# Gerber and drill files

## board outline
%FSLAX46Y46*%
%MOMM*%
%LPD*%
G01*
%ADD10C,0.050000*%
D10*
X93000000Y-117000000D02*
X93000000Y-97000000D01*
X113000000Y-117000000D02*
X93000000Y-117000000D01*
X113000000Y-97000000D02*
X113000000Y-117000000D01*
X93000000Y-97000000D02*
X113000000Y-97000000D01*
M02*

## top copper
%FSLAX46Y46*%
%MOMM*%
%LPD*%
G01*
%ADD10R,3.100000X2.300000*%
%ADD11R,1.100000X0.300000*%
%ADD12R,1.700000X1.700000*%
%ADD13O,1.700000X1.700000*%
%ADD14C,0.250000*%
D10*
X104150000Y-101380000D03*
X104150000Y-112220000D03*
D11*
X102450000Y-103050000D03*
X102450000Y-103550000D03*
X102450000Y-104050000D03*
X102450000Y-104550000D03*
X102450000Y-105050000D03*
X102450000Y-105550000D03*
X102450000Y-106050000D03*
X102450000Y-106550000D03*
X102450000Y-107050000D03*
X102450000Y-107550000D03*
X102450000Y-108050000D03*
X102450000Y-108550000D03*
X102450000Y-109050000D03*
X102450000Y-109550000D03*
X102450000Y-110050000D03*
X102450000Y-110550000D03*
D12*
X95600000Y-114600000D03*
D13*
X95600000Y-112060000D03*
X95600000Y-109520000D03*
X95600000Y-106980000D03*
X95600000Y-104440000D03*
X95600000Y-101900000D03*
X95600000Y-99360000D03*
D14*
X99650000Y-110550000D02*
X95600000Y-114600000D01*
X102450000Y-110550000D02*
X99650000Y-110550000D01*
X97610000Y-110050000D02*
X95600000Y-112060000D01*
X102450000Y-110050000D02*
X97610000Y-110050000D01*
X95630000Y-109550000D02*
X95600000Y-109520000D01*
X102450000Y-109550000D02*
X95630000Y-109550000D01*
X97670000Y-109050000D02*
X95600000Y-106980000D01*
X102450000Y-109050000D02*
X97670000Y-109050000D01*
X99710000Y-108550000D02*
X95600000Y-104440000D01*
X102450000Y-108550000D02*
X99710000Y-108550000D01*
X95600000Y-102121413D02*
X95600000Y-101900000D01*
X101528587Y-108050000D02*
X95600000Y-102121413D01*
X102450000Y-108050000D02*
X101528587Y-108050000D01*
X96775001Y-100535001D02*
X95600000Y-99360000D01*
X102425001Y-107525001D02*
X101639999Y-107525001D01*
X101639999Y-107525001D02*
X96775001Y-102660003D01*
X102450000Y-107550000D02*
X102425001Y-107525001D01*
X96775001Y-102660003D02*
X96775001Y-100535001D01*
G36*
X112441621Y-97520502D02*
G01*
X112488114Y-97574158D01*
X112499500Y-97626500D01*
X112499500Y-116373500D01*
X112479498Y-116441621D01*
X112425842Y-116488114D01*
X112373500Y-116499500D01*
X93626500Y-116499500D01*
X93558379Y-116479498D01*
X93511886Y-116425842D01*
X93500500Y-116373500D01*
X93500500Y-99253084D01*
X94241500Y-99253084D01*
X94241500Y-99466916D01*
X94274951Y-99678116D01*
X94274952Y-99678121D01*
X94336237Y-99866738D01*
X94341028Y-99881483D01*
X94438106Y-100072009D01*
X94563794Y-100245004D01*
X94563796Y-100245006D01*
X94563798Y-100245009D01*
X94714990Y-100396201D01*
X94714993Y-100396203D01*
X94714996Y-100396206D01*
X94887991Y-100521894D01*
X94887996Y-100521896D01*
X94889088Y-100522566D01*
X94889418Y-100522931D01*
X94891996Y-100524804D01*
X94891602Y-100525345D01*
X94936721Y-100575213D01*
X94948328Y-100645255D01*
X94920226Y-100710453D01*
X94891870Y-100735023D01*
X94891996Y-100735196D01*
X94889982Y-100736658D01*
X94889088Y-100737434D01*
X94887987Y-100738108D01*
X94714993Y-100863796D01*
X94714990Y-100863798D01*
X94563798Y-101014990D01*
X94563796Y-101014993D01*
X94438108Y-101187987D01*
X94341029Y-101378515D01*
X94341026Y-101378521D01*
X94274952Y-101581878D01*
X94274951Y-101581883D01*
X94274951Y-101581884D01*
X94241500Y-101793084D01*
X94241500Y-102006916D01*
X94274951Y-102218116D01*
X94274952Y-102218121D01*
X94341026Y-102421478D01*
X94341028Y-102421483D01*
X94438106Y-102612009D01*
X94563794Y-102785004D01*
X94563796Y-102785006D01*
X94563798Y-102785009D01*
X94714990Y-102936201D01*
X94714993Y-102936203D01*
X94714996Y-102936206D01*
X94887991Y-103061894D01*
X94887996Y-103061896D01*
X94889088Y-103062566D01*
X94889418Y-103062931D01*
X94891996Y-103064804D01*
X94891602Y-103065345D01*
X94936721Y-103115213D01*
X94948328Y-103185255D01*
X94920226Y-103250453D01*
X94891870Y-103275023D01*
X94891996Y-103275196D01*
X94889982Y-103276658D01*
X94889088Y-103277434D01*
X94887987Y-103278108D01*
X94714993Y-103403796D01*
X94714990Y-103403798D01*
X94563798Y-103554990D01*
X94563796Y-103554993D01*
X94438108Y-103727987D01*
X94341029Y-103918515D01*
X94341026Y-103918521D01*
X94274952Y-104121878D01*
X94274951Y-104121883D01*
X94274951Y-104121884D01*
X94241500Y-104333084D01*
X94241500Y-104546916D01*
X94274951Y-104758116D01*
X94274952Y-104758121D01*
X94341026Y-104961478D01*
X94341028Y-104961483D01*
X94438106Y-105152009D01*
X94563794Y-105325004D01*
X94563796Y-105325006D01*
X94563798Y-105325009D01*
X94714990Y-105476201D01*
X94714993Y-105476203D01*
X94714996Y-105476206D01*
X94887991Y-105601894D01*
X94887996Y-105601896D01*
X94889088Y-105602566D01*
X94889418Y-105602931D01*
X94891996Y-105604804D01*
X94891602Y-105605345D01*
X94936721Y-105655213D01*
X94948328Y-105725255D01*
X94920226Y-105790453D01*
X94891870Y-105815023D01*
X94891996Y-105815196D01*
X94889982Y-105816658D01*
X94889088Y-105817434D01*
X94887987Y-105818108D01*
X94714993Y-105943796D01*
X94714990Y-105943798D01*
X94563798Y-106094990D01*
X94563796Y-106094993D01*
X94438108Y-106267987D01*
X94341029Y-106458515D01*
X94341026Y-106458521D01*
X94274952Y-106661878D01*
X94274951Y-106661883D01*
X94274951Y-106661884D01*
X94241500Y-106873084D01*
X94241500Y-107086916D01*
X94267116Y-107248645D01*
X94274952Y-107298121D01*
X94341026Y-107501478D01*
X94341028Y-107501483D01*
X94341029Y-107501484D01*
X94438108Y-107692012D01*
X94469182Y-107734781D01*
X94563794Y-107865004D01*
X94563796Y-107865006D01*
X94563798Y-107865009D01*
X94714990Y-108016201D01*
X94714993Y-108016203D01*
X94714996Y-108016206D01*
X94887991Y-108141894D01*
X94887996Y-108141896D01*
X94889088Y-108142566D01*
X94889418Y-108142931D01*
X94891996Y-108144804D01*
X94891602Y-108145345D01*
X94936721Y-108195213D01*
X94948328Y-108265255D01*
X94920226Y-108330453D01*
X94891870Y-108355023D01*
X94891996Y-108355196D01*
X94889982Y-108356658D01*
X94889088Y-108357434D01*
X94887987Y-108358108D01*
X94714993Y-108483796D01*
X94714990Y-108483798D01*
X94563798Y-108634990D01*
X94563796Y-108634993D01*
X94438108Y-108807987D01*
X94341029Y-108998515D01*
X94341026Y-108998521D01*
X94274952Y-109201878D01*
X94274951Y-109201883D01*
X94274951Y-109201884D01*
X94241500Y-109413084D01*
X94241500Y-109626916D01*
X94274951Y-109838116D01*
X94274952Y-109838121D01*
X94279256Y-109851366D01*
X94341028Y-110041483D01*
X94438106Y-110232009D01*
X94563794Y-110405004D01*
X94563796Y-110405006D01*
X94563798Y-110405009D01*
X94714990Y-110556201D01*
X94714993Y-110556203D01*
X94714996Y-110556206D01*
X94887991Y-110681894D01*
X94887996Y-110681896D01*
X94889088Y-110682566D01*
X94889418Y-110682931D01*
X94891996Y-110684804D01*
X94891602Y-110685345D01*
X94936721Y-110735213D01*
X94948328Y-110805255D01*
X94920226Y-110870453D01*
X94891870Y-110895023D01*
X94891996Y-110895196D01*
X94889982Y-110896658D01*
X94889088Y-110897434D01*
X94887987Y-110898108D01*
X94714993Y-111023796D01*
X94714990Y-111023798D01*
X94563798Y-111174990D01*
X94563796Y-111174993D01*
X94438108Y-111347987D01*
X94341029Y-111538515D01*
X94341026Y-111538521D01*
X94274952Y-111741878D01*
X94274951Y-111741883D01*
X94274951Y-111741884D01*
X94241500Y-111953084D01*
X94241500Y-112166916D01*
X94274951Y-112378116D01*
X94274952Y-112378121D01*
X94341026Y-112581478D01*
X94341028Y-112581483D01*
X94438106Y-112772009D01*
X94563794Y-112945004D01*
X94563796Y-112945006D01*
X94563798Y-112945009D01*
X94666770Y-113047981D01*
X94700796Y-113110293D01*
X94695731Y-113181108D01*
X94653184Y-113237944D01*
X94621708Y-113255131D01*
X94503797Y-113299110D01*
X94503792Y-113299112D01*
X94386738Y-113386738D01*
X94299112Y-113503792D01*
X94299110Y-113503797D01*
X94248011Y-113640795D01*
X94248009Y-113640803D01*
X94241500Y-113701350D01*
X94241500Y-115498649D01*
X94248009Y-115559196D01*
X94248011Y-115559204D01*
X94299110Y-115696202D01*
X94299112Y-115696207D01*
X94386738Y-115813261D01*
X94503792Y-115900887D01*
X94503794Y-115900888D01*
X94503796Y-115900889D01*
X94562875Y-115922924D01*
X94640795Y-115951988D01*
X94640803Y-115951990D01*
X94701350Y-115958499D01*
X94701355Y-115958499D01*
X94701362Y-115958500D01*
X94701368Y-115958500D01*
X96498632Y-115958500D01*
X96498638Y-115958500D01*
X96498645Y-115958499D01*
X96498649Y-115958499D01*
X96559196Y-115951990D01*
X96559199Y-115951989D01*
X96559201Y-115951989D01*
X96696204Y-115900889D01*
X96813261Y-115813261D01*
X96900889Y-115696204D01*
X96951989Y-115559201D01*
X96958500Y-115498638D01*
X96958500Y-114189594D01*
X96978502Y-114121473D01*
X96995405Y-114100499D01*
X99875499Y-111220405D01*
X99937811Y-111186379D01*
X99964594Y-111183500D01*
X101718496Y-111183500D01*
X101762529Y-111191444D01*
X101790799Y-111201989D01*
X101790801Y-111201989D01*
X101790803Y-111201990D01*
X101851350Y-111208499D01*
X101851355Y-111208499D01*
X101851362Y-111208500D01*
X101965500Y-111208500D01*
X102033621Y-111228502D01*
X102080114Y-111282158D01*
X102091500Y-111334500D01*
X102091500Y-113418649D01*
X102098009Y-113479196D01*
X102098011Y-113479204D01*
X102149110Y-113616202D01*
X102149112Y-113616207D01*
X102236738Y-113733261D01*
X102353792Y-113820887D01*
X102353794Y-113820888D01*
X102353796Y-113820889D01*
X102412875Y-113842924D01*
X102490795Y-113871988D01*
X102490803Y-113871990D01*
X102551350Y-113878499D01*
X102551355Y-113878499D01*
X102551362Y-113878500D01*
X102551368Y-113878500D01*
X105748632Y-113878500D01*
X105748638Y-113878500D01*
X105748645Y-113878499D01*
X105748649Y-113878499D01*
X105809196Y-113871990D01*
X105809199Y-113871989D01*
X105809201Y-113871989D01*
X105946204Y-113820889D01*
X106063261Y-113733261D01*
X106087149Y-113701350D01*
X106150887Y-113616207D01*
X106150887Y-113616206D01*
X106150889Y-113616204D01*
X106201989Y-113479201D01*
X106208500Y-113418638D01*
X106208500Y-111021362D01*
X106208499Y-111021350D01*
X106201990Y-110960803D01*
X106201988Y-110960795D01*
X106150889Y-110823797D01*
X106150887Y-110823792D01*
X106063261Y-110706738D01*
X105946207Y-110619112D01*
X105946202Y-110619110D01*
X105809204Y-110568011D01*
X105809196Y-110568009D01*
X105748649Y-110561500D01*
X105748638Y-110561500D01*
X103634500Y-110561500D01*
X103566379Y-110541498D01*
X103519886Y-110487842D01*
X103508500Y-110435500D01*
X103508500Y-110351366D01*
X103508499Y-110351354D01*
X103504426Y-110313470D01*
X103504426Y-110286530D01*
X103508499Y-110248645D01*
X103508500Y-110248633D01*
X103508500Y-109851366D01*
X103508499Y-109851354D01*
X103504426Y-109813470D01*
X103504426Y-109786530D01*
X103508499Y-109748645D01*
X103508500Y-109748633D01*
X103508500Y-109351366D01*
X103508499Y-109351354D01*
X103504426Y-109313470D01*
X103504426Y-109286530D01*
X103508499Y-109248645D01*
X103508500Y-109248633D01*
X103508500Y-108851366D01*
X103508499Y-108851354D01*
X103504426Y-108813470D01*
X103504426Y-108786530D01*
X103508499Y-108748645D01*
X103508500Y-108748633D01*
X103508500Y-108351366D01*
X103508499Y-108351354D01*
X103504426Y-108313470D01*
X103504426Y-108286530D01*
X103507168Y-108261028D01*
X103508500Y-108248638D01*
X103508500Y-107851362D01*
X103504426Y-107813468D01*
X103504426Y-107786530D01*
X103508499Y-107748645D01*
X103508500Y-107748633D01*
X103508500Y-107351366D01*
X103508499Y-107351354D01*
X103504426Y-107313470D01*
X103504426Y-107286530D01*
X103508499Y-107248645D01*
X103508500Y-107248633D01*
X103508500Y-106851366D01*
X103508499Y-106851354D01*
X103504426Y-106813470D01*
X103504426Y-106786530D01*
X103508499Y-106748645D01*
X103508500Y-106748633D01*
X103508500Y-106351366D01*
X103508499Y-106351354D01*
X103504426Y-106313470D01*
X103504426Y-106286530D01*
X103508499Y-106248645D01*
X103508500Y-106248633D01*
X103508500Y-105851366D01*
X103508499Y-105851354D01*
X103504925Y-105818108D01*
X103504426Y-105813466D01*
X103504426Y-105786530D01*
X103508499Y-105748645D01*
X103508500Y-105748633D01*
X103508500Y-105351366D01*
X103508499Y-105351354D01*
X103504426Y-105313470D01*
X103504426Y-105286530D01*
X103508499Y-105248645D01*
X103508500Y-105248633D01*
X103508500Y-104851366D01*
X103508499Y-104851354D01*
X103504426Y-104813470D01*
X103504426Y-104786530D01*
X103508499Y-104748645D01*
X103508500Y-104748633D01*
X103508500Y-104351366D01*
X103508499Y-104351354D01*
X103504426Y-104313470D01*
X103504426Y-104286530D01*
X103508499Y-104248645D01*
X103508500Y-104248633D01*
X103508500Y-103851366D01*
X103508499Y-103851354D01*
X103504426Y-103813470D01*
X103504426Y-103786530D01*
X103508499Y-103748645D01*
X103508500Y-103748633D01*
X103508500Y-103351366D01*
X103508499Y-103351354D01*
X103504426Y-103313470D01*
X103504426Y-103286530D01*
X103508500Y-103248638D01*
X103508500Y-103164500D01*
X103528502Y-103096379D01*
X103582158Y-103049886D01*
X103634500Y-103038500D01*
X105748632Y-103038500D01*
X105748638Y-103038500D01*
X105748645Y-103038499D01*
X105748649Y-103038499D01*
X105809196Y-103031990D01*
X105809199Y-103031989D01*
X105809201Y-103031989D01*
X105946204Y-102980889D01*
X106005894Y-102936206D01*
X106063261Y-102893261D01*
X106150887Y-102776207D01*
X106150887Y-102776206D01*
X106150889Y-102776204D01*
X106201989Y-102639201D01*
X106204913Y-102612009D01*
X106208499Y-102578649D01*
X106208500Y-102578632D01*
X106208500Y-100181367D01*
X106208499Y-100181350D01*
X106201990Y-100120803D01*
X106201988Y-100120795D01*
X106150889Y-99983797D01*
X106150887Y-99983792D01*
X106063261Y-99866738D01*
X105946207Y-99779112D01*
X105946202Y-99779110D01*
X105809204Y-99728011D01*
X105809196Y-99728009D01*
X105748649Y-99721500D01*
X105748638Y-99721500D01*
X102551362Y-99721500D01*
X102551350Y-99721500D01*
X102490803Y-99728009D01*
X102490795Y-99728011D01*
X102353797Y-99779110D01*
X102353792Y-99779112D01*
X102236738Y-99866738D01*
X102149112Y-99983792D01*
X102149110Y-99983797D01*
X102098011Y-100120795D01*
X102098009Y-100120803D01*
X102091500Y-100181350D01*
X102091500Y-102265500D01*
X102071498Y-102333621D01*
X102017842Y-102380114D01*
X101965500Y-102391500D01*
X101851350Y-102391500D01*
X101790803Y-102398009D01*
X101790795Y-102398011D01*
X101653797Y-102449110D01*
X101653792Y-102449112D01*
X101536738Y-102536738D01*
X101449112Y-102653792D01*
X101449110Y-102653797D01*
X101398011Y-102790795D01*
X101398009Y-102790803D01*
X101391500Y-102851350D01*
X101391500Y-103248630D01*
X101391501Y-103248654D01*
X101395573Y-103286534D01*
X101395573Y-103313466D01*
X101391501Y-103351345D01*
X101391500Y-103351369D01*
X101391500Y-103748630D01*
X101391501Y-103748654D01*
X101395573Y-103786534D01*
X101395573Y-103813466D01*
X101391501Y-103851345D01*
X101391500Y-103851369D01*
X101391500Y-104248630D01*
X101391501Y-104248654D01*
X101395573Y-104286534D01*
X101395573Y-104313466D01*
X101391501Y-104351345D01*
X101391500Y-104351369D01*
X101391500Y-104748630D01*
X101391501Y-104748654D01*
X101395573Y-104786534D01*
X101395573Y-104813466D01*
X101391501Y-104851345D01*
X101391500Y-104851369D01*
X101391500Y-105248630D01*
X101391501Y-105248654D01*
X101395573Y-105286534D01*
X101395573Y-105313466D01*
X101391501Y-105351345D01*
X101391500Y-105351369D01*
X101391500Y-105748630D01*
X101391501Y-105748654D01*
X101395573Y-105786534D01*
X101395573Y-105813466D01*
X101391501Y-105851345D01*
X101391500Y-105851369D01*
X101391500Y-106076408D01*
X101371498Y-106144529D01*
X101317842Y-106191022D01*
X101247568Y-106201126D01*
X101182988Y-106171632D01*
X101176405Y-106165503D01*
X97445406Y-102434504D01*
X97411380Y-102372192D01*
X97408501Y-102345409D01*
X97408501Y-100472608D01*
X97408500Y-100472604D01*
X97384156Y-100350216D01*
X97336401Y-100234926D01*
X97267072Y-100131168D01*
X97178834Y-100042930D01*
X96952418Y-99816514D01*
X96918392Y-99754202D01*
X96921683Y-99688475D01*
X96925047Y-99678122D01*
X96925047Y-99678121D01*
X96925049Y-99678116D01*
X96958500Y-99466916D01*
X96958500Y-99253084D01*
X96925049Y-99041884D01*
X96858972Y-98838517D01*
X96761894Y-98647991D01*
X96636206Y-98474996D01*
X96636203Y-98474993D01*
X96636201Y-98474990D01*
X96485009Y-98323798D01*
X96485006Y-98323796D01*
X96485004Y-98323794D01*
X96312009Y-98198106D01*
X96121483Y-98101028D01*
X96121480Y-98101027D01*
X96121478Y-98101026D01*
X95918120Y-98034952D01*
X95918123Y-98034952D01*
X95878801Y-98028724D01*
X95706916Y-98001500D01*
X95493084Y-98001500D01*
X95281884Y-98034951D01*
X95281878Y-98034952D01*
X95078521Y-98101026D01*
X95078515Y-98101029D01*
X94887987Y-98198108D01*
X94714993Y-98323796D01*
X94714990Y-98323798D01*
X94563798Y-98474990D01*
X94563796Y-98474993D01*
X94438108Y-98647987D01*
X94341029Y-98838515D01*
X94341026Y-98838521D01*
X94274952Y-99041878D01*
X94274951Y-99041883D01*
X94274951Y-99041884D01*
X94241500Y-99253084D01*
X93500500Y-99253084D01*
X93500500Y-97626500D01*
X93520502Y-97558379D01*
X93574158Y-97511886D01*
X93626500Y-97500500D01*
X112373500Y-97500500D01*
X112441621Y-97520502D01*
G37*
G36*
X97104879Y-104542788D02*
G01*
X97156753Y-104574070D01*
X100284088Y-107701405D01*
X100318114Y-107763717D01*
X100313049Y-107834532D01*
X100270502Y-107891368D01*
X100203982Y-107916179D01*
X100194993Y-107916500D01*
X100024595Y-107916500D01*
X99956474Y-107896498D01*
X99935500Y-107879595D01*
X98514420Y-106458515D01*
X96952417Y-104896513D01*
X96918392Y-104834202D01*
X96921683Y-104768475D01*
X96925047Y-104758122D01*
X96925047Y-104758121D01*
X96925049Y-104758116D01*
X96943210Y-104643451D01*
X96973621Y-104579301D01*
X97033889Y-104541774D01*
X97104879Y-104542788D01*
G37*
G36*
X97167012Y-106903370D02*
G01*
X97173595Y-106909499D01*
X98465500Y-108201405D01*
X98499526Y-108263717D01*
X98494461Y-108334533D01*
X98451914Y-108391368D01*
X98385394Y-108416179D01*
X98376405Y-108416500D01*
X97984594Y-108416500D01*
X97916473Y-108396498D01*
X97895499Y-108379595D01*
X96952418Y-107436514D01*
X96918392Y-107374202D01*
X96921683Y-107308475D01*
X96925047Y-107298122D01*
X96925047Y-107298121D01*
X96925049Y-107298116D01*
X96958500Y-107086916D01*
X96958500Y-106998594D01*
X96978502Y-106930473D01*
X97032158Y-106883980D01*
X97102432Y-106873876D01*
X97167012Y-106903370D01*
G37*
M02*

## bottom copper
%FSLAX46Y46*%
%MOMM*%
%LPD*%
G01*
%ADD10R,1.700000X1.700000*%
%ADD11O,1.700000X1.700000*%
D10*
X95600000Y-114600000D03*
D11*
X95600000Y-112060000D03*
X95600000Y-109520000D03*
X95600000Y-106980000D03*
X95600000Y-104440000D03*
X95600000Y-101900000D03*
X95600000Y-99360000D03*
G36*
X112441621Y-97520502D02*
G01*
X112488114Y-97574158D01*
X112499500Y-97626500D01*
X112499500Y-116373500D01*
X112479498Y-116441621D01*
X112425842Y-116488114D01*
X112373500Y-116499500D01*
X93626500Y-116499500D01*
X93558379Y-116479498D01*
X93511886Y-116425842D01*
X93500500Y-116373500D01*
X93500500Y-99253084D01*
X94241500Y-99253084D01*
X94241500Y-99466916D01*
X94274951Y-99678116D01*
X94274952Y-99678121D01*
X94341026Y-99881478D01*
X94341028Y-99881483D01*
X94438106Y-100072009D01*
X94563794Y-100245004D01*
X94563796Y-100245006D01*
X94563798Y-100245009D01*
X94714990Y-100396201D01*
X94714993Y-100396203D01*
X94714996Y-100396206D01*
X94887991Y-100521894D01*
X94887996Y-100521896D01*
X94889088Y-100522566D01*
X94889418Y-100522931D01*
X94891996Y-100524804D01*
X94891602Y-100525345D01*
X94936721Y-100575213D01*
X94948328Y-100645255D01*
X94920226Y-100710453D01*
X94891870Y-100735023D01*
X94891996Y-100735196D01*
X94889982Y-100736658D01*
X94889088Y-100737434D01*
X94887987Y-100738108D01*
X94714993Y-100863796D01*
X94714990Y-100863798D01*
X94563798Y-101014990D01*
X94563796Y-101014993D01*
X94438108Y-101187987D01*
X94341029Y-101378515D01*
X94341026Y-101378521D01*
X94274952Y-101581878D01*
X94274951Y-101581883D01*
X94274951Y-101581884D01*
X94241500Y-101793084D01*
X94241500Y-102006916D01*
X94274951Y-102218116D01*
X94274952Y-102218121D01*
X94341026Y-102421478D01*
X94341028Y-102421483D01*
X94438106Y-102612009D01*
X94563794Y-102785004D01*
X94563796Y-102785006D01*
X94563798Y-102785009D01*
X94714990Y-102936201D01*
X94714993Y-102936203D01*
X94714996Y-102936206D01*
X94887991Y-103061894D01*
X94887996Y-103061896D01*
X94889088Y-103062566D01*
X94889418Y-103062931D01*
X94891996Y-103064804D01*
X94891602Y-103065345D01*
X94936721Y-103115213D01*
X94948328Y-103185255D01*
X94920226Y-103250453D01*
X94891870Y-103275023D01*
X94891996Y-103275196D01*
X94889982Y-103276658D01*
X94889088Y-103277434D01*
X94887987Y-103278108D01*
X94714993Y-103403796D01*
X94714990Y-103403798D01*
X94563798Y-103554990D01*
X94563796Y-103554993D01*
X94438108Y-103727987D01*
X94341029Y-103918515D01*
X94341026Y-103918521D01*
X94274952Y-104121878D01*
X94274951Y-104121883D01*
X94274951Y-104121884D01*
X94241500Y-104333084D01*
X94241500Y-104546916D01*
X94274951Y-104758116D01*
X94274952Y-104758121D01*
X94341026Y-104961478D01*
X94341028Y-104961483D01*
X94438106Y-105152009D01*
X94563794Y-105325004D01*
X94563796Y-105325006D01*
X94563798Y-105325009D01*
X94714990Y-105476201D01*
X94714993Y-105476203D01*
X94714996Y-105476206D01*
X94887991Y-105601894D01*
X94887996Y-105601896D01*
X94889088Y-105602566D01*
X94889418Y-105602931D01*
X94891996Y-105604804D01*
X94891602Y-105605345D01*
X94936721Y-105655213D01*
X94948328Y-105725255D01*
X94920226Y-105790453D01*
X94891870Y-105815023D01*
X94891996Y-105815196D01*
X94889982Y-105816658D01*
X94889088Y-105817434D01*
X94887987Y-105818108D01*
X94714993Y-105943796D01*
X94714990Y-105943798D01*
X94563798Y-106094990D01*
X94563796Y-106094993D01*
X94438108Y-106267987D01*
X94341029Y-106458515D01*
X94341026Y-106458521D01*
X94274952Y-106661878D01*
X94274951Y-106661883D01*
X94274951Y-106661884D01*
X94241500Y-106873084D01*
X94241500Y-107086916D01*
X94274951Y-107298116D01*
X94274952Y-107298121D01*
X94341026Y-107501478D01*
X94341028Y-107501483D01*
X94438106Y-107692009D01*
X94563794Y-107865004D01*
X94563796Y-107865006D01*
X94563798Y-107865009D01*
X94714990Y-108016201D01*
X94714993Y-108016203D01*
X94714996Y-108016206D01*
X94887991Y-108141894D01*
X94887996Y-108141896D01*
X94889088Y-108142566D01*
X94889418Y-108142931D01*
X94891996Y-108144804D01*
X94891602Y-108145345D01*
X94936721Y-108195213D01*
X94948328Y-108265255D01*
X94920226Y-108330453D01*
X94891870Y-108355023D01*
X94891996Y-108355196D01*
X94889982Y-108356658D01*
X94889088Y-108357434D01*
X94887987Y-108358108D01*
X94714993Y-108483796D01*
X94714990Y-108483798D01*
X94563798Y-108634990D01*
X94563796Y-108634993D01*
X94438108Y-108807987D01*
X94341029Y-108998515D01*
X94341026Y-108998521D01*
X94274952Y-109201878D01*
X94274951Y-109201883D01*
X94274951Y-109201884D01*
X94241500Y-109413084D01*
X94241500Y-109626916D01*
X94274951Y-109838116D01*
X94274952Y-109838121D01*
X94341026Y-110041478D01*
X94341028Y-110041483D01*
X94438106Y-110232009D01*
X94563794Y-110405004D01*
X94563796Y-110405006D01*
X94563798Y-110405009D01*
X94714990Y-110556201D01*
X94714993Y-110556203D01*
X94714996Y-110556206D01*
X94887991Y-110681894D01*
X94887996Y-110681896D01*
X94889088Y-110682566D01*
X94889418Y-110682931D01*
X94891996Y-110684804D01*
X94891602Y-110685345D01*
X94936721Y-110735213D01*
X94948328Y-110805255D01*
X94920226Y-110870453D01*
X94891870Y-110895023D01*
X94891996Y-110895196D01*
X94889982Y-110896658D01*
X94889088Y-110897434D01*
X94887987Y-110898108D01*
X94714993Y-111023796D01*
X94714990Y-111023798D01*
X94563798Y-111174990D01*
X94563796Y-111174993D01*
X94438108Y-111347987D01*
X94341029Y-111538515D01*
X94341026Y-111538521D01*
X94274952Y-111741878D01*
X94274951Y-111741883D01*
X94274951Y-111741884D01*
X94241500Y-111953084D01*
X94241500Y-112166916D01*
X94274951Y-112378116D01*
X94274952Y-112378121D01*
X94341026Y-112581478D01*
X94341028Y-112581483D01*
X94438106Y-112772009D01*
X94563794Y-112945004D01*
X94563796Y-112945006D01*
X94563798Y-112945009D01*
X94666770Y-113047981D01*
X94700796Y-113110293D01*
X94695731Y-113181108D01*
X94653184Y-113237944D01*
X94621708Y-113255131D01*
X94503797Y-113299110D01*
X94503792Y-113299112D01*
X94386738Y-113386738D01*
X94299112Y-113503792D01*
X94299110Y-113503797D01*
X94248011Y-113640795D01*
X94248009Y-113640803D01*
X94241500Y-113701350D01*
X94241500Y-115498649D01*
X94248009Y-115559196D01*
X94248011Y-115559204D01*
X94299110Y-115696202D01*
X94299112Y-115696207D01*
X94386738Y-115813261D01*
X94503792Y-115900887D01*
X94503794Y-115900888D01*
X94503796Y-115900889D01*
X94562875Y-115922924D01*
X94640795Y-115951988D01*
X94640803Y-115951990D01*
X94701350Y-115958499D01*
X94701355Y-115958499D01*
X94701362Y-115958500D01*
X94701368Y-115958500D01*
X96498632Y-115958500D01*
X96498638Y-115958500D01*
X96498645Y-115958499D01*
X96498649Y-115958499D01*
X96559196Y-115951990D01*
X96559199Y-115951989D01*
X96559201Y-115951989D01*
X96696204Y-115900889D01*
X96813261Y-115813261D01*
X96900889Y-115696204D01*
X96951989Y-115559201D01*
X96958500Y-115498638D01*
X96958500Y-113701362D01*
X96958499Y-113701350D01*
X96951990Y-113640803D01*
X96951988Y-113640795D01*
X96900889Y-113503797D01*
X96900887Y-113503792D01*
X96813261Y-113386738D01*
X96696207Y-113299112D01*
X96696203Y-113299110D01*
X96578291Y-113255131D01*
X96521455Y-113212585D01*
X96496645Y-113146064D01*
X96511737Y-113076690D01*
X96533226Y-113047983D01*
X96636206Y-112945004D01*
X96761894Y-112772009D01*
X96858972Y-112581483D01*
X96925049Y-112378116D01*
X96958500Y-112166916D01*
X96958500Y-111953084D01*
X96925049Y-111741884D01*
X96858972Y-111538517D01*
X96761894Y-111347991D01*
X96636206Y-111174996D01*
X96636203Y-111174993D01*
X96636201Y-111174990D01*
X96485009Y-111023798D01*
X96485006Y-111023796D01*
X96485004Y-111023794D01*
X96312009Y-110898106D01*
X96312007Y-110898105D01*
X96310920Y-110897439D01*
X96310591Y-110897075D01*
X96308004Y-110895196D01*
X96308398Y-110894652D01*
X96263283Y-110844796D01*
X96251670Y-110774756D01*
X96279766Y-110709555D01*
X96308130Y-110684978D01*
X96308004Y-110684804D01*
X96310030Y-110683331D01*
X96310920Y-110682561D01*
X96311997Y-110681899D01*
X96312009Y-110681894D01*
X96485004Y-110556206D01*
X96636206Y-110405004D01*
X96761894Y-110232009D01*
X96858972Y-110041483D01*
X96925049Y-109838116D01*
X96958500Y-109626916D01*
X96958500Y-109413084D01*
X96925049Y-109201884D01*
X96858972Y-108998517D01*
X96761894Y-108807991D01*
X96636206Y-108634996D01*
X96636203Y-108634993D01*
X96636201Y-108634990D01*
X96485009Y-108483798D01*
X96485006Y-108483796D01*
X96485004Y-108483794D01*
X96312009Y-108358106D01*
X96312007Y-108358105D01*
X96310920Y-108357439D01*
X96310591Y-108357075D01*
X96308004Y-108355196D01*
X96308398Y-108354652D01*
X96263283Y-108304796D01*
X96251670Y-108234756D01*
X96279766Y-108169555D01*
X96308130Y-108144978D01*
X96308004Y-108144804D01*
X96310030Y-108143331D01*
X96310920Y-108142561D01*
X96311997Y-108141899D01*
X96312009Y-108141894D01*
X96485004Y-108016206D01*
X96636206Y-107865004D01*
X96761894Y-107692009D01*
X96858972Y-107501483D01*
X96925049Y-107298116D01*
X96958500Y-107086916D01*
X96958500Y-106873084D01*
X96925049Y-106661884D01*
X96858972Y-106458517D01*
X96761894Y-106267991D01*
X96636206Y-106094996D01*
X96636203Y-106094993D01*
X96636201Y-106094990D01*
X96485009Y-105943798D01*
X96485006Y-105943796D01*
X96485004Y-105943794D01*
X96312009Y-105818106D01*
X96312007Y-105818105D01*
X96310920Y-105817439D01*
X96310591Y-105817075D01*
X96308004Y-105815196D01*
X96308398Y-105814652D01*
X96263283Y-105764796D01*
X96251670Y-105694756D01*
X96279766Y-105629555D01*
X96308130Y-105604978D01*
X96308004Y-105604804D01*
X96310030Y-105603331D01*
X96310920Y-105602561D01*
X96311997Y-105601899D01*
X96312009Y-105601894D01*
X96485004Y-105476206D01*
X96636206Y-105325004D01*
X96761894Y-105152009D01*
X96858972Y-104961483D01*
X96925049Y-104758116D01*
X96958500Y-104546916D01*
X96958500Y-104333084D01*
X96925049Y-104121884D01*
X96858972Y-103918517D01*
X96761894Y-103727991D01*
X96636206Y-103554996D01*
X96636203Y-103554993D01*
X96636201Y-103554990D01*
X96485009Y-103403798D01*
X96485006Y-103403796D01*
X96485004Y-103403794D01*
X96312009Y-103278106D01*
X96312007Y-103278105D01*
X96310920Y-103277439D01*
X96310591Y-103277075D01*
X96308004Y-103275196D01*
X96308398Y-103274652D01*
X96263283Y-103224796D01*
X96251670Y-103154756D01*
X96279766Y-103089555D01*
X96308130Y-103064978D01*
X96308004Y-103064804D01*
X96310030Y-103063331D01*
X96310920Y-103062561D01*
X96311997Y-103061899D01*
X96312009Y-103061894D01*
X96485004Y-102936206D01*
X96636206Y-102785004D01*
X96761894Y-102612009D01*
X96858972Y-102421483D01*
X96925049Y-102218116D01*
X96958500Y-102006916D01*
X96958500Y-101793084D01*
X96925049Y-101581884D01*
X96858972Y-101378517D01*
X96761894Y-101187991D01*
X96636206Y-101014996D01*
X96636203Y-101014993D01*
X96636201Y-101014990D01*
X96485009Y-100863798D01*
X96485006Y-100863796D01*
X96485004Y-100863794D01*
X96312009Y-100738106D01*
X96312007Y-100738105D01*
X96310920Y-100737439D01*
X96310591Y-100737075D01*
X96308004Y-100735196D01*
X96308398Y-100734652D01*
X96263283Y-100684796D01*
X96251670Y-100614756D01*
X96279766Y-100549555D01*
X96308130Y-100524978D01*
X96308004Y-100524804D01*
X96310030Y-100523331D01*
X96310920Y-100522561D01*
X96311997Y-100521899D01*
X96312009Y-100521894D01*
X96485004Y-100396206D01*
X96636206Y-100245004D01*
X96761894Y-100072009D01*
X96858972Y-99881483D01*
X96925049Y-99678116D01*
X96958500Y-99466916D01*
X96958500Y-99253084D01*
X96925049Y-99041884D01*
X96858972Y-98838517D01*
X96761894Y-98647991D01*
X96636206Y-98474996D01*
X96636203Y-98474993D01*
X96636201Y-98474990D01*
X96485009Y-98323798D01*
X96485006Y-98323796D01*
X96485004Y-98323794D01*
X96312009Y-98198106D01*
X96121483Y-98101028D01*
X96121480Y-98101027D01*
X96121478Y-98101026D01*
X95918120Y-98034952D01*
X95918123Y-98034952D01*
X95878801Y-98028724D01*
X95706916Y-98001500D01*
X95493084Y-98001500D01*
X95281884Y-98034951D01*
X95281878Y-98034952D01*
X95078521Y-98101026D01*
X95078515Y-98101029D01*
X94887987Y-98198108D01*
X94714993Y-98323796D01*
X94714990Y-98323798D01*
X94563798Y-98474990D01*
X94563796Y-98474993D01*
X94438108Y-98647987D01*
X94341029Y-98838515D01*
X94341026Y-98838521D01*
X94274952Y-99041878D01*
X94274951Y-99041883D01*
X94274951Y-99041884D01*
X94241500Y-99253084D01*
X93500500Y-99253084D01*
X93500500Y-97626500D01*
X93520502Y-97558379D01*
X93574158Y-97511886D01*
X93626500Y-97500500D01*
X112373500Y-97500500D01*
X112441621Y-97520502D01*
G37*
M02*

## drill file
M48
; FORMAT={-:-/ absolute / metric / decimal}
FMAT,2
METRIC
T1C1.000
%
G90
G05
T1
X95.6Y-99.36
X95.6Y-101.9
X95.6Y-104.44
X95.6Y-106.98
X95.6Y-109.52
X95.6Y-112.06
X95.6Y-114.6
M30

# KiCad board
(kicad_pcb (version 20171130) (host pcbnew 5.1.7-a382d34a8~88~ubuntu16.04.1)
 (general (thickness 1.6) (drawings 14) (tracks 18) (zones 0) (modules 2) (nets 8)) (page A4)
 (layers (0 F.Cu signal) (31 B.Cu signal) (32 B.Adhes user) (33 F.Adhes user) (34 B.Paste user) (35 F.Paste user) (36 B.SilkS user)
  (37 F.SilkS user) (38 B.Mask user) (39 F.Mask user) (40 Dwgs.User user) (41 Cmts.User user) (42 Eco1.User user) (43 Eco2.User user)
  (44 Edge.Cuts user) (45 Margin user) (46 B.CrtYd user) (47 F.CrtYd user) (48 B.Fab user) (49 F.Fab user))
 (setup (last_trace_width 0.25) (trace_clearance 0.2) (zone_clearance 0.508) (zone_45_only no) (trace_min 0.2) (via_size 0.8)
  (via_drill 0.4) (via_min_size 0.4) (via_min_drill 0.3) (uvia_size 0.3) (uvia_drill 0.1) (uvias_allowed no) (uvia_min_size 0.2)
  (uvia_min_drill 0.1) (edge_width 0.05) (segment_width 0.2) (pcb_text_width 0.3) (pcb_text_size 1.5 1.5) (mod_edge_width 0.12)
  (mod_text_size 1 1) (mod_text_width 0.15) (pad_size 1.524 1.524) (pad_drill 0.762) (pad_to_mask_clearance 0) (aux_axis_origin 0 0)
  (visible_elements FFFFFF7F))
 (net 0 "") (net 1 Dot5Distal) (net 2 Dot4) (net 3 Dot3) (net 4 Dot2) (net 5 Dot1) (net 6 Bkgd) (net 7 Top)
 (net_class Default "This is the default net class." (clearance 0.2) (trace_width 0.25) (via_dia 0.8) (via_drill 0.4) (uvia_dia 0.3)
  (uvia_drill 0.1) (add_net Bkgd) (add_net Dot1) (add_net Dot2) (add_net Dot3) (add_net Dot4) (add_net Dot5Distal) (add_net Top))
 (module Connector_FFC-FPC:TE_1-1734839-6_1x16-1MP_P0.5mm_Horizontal (layer F.Cu) (at 103.8 106.8 90)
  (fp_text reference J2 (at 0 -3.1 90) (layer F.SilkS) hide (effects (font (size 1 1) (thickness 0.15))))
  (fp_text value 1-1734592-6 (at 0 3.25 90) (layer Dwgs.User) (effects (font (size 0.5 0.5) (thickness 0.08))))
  (pad MP smd rect (at 5.42 0.35 90) (size 2.3 3.1) (layers F.Cu F.Paste F.Mask))
  (pad MP smd rect (at -5.42 0.35 90) (size 2.3 3.1) (layers F.Cu F.Paste F.Mask))
  (pad 16 smd rect (at 3.75 -1.35 90) (size 0.3 1.1) (layers F.Cu F.Paste F.Mask))
  (pad 15 smd rect (at 3.25 -1.35 90) (size 0.3 1.1) (layers F.Cu F.Paste F.Mask))
  (pad 14 smd rect (at 2.75 -1.35 90) (size 0.3 1.1) (layers F.Cu F.Paste F.Mask))
  (pad 13 smd rect (at 2.25 -1.35 90) (size 0.3 1.1) (layers F.Cu F.Paste F.Mask))
  (pad 12 smd rect (at 1.75 -1.35 90) (size 0.3 1.1) (layers F.Cu F.Paste F.Mask))
  (pad 11 smd rect (at 1.25 -1.35 90) (size 0.3 1.1) (layers F.Cu F.Paste F.Mask))
  (pad 10 smd rect (at 0.75 -1.35 90) (size 0.3 1.1) (layers F.Cu F.Paste F.Mask))
  (pad 9 smd rect (at 0.25 -1.35 90) (size 0.3 1.1) (layers F.Cu F.Paste F.Mask))
  (pad 8 smd rect (at -0.25 -1.35 90) (size 0.3 1.1) (layers F.Cu F.Paste F.Mask))
  (pad 7 smd rect (at -0.75 -1.35 90) (size 0.3 1.1) (layers F.Cu F.Paste F.Mask) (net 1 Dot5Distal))
  (pad 6 smd rect (at -1.25 -1.35 90) (size 0.3 1.1) (layers F.Cu F.Paste F.Mask) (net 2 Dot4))
  (pad 5 smd rect (at -1.75 -1.35 90) (size 0.3 1.1) (layers F.Cu F.Paste F.Mask) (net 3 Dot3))
  (pad 4 smd rect (at -2.25 -1.35 90) (size 0.3 1.1) (layers F.Cu F.Paste F.Mask) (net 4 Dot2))
  (pad 3 smd rect (at -2.75 -1.35 90) (size 0.3 1.1) (layers F.Cu F.Paste F.Mask) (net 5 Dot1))
  (pad 2 smd rect (at -3.25 -1.35 90) (size 0.3 1.1) (layers F.Cu F.Paste F.Mask) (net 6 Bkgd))
  (pad 1 smd rect (at -3.75 -1.35 90) (size 0.3 1.1) (layers F.Cu F.Paste F.Mask) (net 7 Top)))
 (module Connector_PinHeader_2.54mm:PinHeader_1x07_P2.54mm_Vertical (layer F.Cu) (at 95.6 114.6 180)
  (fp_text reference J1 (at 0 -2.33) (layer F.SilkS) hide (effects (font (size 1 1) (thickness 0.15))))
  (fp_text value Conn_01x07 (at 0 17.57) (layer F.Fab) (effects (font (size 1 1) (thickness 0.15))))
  (pad 1 thru_hole rect (at 0 0 180) (size 1.7 1.7) (drill 1) (layers *.Cu *.Mask) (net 7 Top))
  (pad 2 thru_hole oval (at 0 2.54 180) (size 1.7 1.7) (drill 1) (layers *.Cu *.Mask) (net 6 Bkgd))
  (pad 3 thru_hole oval (at 0 5.08 180) (size 1.7 1.7) (drill 1) (layers *.Cu *.Mask) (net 5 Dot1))
  (pad 4 thru_hole oval (at 0 7.62 180) (size 1.7 1.7) (drill 1) (layers *.Cu *.Mask) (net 4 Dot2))
  (pad 5 thru_hole oval (at 0 10.16 180) (size 1.7 1.7) (drill 1) (layers *.Cu *.Mask) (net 3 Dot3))
  (pad 6 thru_hole oval (at 0 12.7 180) (size 1.7 1.7) (drill 1) (layers *.Cu *.Mask) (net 2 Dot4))
  (pad 7 thru_hole oval (at 0 15.24 180) (size 1.7 1.7) (drill 1) (layers *.Cu *.Mask) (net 1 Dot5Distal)))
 (gr_line (start 93 117) (end 93 97) (layer Edge.Cuts) (width 0.05))
 (gr_line (start 113 117) (end 93 117) (layer Edge.Cuts) (width 0.05))
 (gr_line (start 113 97) (end 113 117) (layer Edge.Cuts) (width 0.05))
 (gr_line (start 93 97) (end 113 97) (layer Edge.Cuts) (width 0.05))
 (segment (start 99.65 110.55) (end 95.6 114.6) (width 0.25) (layer F.Cu) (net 7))
 (segment (start 102.45 110.55) (end 99.65 110.55) (width 0.25) (layer F.Cu) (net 7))
 (segment (start 97.61 110.05) (end 95.6 112.06) (width 0.25) (layer F.Cu) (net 6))
 (segment (start 102.45 110.05) (end 97.61 110.05) (width 0.25) (layer F.Cu) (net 6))
 (segment (start 95.63 109.55) (end 95.6 109.52) (width 0.25) (layer F.Cu) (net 5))
 (segment (start 102.45 109.55) (end 95.63 109.55) (width 0.25) (layer F.Cu) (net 5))
 (segment (start 97.67 109.05) (end 95.6 106.98) (width 0.25) (layer F.Cu) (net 4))
 (segment (start 102.45 109.05) (end 97.67 109.05) (width 0.25) (layer F.Cu) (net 4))
 (segment (start 99.71 108.55) (end 95.6 104.44) (width 0.25) (layer F.Cu) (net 3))
 (segment (start 102.45 108.55) (end 99.71 108.55) (width 0.25) (layer F.Cu) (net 3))
 (segment (start 95.6 102.121413) (end 95.6 101.9) (width 0.25) (layer F.Cu) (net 2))
 (segment (start 101.528587 108.05) (end 95.6 102.121413) (width 0.25) (layer F.Cu) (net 2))
 (segment (start 102.45 108.05) (end 101.528587 108.05) (width 0.25) (layer F.Cu) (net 2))
 (segment (start 96.775001 100.535001) (end 95.6 99.36) (width 0.25) (layer F.Cu) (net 1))
 (segment (start 102.425001 107.525001) (end 101.639999 107.525001) (width 0.25) (layer F.Cu) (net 1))
 (segment (start 101.639999 107.525001) (end 96.775001 102.660003) (width 0.25) (layer F.Cu) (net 1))
 (segment (start 102.45 107.55) (end 102.425001 107.525001) (width 0.25) (layer F.Cu) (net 1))
 (segment (start 96.775001 102.660003) (end 96.775001 100.535001) (width 0.25) (layer F.Cu) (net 1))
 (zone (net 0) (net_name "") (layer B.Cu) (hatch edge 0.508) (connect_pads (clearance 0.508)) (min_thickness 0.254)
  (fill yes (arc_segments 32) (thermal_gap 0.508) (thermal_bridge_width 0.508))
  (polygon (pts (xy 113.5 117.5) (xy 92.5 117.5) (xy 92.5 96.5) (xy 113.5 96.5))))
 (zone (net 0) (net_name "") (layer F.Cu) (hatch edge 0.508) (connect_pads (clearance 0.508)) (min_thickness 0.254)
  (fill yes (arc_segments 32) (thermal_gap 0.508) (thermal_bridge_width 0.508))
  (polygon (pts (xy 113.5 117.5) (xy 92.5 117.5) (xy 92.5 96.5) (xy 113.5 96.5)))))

